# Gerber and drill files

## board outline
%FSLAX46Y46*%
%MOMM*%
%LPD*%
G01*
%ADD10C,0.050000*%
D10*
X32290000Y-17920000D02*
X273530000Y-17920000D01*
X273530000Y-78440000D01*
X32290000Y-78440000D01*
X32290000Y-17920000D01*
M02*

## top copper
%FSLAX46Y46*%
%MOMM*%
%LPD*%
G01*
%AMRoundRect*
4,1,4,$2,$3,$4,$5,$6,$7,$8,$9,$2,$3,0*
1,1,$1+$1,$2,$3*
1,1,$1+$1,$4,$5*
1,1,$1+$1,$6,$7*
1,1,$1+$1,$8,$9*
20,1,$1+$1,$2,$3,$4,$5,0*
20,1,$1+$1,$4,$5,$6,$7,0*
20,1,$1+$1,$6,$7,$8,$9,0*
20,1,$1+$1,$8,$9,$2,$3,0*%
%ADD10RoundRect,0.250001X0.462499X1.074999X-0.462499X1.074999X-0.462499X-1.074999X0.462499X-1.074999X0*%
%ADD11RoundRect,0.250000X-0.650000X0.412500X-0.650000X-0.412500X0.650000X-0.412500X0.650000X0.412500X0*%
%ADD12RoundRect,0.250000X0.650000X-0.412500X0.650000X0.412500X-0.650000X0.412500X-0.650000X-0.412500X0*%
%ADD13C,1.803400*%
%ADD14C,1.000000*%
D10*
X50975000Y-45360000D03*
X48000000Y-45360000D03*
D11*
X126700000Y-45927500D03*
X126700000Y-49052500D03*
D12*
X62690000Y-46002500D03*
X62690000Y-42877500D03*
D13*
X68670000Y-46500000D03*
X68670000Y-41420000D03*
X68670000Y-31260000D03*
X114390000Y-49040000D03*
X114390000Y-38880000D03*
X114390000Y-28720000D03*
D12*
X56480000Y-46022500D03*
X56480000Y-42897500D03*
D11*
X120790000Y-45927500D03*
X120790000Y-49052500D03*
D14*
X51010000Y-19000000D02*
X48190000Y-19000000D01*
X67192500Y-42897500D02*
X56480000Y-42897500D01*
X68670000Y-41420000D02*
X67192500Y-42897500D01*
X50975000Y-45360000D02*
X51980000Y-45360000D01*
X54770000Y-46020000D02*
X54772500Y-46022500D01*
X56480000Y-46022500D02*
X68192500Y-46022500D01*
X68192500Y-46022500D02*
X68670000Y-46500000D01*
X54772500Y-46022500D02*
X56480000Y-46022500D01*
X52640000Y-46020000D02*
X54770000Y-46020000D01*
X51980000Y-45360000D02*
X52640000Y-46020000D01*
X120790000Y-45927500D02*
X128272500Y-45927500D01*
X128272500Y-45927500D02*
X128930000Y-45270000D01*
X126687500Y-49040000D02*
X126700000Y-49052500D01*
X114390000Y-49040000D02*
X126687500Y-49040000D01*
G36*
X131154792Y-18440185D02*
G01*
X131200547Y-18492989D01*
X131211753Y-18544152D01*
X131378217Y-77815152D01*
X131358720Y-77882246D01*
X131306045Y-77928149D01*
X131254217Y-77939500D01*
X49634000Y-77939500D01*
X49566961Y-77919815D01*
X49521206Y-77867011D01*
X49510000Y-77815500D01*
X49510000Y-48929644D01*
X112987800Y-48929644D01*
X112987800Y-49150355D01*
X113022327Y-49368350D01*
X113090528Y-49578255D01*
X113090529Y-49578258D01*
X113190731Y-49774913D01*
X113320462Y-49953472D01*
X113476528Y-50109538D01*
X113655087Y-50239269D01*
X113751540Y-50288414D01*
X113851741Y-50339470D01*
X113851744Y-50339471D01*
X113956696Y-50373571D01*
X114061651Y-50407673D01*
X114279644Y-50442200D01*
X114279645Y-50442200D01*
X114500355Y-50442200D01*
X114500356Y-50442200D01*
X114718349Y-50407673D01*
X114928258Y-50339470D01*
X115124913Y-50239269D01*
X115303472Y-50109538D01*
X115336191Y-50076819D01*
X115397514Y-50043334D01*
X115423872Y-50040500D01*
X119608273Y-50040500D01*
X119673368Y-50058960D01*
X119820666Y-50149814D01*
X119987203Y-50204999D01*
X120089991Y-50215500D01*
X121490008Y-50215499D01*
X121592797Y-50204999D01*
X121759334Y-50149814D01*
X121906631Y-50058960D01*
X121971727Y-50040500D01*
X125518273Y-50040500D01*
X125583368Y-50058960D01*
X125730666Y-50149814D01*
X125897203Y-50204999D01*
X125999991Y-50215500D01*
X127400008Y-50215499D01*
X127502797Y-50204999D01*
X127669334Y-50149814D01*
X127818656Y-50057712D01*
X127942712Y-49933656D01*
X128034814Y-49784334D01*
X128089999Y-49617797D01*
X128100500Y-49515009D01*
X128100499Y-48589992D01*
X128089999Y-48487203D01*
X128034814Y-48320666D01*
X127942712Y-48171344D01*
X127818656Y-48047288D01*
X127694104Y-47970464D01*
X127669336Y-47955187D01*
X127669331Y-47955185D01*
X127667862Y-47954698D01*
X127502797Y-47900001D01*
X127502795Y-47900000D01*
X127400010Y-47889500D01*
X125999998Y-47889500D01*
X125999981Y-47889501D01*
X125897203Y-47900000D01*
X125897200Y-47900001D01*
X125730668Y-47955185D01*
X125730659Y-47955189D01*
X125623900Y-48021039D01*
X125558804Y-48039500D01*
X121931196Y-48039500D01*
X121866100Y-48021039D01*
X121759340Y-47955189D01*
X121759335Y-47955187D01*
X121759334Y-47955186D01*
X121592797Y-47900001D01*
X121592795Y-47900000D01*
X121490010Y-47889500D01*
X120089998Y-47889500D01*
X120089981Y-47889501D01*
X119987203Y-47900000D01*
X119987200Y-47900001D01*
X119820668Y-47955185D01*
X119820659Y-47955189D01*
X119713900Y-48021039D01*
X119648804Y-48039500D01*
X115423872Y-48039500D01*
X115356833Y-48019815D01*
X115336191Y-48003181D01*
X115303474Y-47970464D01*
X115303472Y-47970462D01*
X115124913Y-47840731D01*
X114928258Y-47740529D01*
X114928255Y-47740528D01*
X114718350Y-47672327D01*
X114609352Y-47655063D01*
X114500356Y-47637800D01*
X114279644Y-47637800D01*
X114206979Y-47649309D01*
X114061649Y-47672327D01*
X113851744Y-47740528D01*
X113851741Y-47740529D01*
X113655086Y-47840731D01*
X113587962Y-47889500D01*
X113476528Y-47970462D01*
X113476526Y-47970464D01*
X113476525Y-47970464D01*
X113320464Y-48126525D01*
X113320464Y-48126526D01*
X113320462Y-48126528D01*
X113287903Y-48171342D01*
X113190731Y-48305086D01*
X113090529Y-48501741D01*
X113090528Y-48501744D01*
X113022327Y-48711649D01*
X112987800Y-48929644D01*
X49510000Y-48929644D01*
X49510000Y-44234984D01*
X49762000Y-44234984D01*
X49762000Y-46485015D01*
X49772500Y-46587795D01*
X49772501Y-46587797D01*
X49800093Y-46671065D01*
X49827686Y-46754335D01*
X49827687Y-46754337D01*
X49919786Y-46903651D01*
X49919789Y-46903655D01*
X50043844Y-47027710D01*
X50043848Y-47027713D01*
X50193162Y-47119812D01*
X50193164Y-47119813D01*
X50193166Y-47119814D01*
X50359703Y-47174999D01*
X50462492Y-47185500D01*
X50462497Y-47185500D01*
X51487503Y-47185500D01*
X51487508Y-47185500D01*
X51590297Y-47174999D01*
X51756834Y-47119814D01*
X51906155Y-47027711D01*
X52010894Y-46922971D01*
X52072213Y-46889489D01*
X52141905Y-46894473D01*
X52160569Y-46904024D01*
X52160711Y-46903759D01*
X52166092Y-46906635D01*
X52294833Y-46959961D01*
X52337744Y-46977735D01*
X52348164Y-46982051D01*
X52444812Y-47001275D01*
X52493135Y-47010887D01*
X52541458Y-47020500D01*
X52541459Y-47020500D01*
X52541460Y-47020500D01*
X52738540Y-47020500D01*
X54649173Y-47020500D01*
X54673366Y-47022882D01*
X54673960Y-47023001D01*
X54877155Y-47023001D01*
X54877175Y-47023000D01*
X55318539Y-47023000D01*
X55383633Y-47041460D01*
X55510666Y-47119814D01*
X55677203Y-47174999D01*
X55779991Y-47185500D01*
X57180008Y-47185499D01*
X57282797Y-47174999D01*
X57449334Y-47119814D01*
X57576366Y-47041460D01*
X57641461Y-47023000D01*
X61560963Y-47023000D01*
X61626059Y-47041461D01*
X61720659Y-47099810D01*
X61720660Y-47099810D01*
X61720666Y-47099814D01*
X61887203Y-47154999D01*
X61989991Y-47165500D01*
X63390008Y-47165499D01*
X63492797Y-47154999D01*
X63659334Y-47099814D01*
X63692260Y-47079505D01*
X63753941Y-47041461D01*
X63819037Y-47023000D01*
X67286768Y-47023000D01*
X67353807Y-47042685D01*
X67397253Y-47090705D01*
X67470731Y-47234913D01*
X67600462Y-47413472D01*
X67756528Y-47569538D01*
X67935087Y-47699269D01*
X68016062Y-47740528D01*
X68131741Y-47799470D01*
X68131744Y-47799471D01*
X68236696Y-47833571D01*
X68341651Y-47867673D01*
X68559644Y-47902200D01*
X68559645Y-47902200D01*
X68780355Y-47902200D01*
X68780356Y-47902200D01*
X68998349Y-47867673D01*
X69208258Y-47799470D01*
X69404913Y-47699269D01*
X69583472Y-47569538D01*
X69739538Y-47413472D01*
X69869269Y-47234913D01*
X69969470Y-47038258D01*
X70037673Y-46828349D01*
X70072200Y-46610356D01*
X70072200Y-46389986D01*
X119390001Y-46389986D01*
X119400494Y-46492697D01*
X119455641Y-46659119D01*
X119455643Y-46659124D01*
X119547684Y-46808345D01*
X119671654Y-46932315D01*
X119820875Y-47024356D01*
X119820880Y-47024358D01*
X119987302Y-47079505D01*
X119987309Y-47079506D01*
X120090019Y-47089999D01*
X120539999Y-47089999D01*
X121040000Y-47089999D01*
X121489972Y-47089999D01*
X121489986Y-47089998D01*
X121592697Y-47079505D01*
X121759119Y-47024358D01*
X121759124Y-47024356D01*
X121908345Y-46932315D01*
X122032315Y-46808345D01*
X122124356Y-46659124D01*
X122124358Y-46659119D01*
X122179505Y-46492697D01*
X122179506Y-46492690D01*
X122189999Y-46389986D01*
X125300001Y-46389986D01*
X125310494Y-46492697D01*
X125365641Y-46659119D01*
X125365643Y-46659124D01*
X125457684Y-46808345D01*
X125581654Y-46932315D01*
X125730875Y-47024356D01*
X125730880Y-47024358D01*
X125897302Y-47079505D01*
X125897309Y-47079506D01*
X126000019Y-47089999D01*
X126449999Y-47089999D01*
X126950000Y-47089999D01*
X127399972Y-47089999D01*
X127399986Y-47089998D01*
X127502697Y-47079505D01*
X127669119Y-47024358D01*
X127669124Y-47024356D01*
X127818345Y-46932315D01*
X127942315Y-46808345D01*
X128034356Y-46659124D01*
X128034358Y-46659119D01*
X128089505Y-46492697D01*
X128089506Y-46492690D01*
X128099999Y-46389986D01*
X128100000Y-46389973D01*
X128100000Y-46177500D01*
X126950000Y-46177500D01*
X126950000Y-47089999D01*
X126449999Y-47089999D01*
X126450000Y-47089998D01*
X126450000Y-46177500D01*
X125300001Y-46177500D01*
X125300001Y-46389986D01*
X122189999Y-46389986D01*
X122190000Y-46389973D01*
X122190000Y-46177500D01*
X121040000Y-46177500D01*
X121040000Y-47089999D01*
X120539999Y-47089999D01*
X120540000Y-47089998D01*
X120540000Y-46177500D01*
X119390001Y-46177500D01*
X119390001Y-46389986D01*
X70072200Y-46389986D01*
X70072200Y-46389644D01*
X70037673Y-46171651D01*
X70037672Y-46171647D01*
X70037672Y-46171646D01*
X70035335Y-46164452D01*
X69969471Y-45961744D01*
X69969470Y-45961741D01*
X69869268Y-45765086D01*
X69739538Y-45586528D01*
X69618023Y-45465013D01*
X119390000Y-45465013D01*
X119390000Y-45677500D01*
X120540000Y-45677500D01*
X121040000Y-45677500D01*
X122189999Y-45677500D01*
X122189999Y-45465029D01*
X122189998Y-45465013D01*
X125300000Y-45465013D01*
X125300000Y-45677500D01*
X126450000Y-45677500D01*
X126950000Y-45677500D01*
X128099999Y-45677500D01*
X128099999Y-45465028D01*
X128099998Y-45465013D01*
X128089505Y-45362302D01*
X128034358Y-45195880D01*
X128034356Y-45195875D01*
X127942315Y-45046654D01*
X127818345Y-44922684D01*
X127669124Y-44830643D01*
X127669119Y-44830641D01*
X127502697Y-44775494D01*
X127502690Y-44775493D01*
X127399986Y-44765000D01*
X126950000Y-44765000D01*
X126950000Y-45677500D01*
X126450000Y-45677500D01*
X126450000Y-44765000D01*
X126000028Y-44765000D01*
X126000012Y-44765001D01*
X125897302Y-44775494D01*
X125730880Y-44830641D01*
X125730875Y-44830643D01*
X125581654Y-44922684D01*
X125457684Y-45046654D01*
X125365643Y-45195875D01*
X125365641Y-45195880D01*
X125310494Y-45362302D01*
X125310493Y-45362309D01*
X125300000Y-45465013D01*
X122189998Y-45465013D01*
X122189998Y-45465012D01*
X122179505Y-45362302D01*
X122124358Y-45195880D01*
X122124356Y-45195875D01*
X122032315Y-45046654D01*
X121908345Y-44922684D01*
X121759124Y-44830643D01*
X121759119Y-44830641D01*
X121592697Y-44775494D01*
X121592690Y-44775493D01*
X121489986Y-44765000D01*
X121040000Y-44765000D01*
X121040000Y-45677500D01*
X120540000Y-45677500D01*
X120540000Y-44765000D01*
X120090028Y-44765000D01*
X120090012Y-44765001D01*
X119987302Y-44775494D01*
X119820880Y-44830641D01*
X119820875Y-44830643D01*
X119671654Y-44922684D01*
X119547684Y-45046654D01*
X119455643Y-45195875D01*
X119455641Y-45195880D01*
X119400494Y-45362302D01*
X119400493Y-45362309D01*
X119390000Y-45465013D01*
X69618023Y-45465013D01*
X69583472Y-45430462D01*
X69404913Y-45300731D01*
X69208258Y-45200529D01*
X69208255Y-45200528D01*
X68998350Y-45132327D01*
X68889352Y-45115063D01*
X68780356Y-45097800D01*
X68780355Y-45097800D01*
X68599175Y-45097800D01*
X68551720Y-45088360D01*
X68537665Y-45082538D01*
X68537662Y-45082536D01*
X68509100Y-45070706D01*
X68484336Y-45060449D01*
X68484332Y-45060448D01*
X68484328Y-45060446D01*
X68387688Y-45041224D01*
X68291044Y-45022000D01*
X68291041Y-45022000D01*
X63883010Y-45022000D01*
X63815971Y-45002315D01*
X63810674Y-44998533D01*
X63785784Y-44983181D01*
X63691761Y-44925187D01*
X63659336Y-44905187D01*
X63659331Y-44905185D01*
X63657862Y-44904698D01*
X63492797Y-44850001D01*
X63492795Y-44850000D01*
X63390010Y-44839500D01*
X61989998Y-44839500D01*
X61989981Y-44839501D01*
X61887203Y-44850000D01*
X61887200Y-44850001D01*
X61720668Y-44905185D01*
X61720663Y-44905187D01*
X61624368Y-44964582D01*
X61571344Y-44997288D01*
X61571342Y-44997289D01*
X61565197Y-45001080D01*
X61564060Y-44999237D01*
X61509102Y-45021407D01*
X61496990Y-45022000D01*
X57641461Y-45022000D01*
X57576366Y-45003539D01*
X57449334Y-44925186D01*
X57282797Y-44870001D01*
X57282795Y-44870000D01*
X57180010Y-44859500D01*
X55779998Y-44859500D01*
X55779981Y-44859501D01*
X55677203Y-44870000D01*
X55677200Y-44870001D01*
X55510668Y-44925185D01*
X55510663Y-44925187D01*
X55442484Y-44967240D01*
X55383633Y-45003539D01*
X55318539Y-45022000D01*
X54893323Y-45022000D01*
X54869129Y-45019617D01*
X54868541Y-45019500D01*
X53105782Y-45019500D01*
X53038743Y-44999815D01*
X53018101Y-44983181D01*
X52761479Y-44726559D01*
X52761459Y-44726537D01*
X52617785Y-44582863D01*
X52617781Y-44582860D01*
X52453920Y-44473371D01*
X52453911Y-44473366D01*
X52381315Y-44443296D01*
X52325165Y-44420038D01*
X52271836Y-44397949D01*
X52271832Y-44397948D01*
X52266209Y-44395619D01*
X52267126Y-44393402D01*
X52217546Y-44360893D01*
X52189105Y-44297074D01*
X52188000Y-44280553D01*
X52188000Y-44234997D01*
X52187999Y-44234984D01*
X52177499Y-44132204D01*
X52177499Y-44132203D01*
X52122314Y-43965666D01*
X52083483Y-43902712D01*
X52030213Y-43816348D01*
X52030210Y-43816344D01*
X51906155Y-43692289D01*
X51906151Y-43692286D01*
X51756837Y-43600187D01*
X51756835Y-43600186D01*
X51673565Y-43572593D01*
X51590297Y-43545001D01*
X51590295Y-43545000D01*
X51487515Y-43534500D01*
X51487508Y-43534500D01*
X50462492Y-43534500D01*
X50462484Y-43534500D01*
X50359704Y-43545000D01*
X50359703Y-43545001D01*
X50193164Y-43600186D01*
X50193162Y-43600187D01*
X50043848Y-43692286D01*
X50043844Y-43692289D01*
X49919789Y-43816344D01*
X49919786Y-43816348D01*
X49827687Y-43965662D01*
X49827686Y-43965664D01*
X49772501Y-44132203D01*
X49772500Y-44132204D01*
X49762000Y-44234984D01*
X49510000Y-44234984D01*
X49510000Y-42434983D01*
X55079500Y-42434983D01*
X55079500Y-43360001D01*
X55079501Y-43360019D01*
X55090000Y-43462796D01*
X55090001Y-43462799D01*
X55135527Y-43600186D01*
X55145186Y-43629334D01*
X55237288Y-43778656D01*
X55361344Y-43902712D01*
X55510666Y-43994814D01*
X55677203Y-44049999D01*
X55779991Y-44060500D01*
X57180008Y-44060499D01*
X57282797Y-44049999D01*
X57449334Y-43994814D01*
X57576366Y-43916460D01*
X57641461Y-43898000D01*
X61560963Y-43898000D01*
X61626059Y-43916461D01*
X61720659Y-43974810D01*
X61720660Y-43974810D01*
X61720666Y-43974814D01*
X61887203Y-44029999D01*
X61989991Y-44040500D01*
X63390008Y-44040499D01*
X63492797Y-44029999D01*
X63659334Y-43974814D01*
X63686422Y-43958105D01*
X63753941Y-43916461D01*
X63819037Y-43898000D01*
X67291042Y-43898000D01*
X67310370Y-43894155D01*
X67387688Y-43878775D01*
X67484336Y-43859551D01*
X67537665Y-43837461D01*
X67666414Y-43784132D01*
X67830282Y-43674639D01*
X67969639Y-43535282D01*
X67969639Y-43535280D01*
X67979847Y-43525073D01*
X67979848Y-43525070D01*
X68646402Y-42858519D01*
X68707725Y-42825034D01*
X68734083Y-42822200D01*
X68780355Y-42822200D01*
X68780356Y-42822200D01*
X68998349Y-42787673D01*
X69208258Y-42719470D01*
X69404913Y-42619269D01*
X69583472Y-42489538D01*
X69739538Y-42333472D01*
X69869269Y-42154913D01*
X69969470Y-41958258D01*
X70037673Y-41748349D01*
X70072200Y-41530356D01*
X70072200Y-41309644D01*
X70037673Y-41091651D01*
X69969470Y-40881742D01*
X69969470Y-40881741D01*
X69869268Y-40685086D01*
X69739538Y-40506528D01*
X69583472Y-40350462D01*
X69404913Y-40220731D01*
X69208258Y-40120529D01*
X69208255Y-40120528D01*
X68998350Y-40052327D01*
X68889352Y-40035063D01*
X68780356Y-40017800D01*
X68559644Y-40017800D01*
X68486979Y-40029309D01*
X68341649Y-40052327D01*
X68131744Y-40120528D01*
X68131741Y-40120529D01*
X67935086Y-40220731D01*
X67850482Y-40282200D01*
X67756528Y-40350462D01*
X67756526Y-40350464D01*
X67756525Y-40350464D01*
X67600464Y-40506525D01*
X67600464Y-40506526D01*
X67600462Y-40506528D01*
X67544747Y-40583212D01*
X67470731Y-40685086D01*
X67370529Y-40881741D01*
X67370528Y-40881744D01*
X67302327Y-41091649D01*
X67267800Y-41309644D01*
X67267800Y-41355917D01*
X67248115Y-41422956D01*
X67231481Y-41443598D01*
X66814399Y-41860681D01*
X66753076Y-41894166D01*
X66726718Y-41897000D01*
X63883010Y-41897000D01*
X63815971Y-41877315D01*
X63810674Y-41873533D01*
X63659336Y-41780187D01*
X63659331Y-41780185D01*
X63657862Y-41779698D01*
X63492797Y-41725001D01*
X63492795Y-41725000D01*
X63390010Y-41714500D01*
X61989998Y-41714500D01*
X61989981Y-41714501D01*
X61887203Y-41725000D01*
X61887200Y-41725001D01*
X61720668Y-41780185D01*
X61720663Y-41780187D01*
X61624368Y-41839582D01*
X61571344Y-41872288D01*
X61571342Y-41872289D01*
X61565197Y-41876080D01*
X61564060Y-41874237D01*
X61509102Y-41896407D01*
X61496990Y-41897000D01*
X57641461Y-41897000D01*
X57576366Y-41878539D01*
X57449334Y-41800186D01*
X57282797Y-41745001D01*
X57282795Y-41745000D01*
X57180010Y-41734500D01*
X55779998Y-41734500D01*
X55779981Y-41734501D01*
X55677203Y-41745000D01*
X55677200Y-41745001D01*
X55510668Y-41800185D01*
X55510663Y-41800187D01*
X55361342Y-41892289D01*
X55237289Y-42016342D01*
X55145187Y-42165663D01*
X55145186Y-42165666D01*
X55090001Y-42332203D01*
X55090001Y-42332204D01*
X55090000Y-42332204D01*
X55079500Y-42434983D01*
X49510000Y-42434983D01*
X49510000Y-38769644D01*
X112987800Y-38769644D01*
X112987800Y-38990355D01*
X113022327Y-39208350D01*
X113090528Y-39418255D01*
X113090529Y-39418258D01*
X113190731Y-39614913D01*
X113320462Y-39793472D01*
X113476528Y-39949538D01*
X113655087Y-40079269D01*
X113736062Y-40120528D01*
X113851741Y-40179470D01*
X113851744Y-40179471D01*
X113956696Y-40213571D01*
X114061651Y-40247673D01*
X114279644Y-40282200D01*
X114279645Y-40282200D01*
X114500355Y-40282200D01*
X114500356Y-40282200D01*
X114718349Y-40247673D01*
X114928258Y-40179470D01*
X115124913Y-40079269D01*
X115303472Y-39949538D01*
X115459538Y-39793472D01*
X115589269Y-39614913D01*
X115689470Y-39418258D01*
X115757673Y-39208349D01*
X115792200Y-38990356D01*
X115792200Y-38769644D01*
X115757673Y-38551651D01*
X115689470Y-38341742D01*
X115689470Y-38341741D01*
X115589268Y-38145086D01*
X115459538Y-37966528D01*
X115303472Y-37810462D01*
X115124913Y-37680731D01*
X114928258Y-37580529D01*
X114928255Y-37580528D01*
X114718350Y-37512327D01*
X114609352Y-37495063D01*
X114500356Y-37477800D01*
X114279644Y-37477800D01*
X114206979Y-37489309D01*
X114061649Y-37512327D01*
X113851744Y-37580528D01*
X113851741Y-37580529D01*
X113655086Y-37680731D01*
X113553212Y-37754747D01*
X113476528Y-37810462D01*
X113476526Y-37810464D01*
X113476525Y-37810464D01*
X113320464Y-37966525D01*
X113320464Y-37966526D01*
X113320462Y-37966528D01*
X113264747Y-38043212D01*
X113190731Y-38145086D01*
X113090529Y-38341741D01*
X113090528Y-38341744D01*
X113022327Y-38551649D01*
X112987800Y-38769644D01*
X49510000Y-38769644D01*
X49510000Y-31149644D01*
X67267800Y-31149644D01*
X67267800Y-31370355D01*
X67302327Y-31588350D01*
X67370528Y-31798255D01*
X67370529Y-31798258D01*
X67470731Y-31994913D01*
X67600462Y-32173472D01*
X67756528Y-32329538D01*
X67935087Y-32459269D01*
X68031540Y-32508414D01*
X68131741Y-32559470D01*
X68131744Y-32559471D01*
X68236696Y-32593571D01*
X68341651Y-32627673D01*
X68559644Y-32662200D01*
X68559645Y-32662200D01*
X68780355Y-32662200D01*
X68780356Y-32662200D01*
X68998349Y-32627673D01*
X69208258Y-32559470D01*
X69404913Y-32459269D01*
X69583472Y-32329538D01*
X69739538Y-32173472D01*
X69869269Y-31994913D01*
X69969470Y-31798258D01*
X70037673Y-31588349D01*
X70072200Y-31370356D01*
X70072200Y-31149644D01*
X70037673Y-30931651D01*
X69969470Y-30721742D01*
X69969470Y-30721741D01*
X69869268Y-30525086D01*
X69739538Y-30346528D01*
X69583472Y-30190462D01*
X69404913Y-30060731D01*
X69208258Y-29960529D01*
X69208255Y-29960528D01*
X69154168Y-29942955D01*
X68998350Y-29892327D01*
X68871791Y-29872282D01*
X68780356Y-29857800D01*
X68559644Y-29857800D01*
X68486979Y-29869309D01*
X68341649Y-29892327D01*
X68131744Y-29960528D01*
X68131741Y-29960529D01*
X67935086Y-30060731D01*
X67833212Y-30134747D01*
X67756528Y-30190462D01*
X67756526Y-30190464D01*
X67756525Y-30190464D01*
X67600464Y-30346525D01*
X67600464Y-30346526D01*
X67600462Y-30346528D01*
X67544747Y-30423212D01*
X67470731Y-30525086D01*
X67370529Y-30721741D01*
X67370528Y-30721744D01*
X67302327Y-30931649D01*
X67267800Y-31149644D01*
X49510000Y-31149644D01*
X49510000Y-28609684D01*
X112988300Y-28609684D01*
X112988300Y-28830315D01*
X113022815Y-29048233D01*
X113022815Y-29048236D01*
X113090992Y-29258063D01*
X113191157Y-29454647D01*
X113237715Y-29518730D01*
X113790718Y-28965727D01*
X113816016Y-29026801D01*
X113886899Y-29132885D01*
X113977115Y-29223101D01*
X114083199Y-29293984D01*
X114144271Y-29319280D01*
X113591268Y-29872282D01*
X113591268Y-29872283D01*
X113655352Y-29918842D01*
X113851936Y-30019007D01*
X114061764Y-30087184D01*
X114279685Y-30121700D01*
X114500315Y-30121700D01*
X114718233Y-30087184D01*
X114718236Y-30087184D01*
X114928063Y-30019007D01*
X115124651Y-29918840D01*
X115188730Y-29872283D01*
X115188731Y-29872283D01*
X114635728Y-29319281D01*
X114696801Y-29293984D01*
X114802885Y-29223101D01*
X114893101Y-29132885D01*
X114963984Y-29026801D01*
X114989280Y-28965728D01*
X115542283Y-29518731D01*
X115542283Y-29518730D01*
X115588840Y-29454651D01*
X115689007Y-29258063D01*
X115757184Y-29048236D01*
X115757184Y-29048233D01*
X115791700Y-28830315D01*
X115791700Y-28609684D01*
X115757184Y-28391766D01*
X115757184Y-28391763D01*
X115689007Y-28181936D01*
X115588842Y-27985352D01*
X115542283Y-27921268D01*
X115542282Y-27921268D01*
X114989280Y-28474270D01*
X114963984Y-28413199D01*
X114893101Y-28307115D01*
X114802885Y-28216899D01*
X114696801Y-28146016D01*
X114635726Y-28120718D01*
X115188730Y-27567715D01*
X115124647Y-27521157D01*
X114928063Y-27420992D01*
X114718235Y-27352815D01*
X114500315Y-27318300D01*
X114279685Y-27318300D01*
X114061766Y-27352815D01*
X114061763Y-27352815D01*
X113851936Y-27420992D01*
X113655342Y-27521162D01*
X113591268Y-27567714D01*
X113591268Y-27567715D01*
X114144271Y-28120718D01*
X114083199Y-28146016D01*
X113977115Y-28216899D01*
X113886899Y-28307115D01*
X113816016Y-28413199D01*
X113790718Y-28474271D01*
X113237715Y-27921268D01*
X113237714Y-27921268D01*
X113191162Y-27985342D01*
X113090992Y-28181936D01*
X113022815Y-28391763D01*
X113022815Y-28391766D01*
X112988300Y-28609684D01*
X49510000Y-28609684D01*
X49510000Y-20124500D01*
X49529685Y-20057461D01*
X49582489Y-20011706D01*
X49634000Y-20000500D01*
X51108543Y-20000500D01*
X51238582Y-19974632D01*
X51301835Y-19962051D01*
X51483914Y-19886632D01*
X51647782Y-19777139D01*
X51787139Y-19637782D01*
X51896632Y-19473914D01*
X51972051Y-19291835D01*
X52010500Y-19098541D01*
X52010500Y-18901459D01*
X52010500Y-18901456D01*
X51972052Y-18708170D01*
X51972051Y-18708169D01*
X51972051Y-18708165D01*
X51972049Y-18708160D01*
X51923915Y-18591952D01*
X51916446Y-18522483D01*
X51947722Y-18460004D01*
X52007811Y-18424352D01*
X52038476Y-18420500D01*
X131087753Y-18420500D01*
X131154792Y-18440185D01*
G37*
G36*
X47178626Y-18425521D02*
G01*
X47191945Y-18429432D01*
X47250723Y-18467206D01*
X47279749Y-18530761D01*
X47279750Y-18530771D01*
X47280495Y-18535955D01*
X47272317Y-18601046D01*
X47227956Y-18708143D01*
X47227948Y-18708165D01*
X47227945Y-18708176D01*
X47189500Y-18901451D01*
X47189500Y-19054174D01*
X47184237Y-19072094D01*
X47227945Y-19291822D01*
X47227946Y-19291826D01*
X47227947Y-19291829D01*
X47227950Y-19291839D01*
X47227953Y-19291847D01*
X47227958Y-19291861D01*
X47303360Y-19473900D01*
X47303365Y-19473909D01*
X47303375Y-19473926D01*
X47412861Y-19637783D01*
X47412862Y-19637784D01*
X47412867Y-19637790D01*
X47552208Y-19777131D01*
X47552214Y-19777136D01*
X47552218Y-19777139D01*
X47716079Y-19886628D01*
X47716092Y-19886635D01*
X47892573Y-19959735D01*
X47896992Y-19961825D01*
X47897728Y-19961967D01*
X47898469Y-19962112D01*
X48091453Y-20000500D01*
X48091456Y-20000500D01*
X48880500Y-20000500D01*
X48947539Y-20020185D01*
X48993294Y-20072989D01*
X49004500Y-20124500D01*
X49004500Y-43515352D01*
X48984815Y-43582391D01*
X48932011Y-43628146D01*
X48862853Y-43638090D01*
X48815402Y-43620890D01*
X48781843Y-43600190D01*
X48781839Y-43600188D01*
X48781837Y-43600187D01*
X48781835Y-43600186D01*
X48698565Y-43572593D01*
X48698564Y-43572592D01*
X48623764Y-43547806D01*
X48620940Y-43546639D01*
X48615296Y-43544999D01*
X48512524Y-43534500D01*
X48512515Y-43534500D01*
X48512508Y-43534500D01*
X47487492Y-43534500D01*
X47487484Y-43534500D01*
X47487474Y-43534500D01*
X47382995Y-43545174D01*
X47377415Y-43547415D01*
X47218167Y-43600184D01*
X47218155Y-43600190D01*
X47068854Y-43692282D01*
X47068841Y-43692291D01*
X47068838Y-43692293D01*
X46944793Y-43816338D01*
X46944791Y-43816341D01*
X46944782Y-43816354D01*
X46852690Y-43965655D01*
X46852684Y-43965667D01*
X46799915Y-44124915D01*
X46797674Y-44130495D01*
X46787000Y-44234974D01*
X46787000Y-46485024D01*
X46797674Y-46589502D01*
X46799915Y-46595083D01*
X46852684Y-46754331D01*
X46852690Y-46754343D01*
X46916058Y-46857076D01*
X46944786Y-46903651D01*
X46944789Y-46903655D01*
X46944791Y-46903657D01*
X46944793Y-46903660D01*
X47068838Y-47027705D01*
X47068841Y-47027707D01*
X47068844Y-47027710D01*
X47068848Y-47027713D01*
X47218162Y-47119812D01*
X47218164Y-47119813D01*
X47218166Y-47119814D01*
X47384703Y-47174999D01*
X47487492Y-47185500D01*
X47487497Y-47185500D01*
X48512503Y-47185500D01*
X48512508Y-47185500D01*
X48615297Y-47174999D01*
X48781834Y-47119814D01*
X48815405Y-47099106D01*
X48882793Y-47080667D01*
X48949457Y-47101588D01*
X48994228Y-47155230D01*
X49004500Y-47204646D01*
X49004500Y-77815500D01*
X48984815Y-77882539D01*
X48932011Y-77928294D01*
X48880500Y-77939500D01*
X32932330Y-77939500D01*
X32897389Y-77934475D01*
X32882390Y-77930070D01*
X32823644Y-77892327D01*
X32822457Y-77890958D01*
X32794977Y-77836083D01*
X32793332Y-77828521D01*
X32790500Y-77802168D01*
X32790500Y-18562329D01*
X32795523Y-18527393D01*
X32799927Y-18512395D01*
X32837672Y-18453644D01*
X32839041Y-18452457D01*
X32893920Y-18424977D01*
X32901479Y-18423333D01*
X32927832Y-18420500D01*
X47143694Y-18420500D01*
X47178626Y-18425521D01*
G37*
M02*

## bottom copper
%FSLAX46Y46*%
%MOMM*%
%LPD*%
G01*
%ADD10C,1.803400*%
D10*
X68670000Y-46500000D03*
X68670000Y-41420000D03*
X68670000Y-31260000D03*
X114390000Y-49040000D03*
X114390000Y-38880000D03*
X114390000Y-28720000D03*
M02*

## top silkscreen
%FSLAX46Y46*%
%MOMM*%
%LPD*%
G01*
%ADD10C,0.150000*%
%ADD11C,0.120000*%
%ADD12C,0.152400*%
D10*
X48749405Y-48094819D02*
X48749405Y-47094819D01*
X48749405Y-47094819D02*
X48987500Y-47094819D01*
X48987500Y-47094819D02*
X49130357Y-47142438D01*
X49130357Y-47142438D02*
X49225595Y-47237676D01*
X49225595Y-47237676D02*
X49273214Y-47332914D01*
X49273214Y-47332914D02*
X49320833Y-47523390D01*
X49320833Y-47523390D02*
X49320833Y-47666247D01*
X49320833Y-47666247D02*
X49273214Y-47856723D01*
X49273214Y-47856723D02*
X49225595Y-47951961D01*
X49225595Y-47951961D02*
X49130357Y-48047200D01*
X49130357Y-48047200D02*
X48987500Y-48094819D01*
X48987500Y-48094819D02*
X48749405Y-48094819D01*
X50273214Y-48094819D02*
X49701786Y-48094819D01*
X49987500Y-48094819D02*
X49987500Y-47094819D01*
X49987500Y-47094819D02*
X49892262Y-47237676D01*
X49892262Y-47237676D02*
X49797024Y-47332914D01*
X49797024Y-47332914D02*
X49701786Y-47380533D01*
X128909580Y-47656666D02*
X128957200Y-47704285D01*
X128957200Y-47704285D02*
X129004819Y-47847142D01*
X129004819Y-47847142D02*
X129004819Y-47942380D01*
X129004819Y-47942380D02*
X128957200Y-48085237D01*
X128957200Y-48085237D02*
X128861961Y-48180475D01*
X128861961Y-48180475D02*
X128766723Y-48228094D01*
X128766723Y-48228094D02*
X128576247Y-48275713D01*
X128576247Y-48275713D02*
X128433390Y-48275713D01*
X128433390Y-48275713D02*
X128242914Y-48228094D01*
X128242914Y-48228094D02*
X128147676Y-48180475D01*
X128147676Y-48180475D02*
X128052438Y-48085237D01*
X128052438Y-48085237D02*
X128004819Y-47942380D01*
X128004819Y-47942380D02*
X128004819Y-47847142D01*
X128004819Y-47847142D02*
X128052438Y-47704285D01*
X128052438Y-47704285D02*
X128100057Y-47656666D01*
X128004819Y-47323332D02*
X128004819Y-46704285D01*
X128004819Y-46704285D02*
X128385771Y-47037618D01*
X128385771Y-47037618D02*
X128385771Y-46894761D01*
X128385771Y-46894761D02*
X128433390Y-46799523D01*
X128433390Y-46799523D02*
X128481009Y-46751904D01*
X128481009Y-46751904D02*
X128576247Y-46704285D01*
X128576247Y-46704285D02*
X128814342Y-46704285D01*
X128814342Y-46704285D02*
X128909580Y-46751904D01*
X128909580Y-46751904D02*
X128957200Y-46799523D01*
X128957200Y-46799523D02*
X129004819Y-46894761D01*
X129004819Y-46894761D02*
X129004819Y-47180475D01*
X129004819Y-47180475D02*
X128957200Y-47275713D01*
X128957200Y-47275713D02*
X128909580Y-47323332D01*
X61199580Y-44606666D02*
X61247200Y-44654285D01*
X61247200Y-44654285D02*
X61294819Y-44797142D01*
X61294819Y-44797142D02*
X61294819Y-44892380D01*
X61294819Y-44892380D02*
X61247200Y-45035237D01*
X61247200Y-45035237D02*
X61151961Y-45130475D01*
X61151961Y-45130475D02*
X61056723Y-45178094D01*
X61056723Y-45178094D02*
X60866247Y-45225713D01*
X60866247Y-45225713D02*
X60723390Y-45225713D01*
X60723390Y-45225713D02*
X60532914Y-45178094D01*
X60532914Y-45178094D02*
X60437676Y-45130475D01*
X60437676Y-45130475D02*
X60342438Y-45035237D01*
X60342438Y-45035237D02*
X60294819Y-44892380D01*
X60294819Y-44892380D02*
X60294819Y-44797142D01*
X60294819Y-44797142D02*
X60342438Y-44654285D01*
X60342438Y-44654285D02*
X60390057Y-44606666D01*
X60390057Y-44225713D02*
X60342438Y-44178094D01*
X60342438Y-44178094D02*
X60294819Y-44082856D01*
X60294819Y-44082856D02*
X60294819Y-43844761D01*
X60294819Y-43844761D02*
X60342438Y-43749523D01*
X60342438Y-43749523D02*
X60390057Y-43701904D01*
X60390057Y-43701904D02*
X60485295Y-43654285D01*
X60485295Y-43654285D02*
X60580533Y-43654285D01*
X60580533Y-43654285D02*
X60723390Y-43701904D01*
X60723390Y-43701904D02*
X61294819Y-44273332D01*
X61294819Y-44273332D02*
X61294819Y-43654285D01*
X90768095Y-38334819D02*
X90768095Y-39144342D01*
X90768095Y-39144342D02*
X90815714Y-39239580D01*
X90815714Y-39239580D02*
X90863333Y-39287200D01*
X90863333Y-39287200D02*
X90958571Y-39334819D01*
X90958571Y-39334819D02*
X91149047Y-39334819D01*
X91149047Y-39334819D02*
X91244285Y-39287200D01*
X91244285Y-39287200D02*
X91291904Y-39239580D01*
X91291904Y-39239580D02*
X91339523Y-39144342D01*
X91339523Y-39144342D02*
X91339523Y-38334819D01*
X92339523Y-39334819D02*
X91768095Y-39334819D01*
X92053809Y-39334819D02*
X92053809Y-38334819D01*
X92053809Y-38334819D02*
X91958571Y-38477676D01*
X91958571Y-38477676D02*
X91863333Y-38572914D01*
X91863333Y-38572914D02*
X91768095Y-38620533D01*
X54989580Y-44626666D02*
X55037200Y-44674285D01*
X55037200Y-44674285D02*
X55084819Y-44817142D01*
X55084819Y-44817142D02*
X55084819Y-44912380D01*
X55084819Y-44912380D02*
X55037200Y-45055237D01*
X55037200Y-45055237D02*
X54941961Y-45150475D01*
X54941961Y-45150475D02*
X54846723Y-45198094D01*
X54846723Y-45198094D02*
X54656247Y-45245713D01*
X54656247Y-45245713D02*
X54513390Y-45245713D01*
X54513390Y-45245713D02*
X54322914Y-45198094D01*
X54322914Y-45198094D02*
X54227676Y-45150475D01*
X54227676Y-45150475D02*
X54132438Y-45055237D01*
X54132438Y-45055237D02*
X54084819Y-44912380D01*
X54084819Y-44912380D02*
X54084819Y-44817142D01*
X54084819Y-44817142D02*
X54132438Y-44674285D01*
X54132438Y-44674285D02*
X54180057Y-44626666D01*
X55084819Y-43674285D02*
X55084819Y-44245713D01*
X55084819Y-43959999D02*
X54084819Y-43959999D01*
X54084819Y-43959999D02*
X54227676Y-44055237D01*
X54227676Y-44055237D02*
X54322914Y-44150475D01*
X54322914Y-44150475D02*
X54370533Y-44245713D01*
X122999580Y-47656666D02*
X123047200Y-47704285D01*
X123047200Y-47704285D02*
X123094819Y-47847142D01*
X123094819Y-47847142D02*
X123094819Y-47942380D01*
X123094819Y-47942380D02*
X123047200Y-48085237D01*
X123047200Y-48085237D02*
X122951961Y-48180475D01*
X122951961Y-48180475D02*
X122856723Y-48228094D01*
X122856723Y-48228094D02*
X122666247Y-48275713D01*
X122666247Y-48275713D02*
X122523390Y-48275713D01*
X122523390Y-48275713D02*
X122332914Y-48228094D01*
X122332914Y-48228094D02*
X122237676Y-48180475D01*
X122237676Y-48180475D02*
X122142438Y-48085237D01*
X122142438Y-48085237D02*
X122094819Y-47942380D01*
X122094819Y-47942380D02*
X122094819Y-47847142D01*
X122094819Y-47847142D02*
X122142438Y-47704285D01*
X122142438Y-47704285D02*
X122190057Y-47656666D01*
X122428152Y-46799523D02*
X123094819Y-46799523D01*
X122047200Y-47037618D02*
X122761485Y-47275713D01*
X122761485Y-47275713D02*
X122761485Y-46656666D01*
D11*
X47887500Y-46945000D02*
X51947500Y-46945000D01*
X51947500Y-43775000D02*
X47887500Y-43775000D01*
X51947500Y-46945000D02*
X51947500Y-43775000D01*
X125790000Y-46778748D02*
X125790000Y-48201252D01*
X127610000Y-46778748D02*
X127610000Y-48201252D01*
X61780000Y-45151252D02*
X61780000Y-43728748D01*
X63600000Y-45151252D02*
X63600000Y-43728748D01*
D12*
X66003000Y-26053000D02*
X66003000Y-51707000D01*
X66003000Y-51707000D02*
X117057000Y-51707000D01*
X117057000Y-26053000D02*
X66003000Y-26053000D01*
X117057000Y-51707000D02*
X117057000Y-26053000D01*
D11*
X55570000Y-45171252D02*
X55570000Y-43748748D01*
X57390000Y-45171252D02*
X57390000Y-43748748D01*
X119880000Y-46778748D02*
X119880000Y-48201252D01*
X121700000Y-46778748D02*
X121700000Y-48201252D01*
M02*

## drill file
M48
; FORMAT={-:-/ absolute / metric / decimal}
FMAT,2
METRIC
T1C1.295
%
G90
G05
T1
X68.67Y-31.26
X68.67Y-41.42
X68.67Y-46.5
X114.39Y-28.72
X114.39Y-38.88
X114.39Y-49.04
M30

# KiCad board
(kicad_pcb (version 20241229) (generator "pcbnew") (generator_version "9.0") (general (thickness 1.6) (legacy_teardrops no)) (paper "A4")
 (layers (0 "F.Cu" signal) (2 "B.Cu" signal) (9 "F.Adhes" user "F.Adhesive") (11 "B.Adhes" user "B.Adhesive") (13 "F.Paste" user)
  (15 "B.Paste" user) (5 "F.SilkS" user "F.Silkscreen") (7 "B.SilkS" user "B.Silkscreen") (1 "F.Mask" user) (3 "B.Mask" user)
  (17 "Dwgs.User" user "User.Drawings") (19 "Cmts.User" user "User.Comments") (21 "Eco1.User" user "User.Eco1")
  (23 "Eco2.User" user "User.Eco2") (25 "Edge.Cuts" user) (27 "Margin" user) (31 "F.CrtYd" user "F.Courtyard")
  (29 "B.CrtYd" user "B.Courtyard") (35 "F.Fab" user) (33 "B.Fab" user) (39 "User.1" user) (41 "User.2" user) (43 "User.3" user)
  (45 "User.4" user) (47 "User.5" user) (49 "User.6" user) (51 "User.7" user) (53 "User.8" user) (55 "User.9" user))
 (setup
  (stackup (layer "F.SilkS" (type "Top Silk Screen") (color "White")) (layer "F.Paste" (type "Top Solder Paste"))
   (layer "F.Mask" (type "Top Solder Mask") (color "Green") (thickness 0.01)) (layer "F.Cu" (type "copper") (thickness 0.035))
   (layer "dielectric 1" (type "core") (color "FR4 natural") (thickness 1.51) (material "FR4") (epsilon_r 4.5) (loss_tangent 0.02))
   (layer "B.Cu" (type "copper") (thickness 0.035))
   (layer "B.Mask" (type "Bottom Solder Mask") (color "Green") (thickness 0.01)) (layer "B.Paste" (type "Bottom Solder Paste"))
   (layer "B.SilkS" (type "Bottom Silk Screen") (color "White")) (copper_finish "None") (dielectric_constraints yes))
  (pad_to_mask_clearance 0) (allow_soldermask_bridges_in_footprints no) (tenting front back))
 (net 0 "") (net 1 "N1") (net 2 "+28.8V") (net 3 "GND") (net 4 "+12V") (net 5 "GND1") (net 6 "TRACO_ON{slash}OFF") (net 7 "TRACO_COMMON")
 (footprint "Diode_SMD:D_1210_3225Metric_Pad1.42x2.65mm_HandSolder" (layer "F.Cu") (at 49.4875 45.36 180)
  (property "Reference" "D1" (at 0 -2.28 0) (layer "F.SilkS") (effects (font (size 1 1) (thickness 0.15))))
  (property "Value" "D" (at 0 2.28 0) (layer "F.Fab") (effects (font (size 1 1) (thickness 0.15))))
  (fp_line (start 1.6 -1.585) (end -2.46 -1.585) (stroke (width 0.12) (type solid)) (layer "F.SilkS"))
  (fp_line (start -2.46 1.585) (end 1.6 1.585) (stroke (width 0.12) (type solid)) (layer "F.SilkS"))
  (fp_line (start -2.46 -1.585) (end -2.46 1.585) (stroke (width 0.12) (type solid)) (layer "F.SilkS"))
  (pad "1" smd roundrect (at -1.4875 0 180) (size 1.425 2.65) (layers "F.Cu" "F.Mask" "F.Paste") (roundrect_rratio 0.175439) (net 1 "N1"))
  (pad "2" smd roundrect (at 1.4875 0 180) (size 1.425 2.65) (layers "F.Cu" "F.Mask" "F.Paste") (roundrect_rratio 0.175439) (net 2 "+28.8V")))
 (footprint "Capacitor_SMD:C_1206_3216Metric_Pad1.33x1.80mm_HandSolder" (layer "F.Cu") (at 126.7 47.49 -90)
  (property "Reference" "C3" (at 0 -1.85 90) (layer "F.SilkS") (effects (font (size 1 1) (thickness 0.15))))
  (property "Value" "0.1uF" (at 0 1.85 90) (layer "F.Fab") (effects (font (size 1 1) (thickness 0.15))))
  (fp_line (start -0.711252 0.91) (end 0.711252 0.91) (stroke (width 0.12) (type solid)) (layer "F.SilkS"))
  (fp_line (start -0.711252 -0.91) (end 0.711252 -0.91) (stroke (width 0.12) (type solid)) (layer "F.SilkS"))
  (pad "1" smd roundrect (at -1.5625 0 270) (size 1.325 1.8) (layers "F.Cu" "F.Mask" "F.Paste") (roundrect_rratio 0.188679) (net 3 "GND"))
  (pad "2" smd roundrect (at 1.5625 0 270) (size 1.325 1.8) (layers "F.Cu" "F.Mask" "F.Paste") (roundrect_rratio 0.188679) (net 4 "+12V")))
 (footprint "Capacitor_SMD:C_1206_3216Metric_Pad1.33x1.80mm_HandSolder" (layer "F.Cu") (at 62.69 44.44 90)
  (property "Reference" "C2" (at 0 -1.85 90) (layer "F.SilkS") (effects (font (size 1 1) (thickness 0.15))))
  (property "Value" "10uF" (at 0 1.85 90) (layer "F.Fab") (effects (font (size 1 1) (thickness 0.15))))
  (fp_line (start -0.711252 -0.91) (end 0.711252 -0.91) (stroke (width 0.12) (type solid)) (layer "F.SilkS"))
  (fp_line (start -0.711252 0.91) (end 0.711252 0.91) (stroke (width 0.12) (type solid)) (layer "F.SilkS"))
  (pad "1" smd roundrect (at -1.5625 0 90) (size 1.325 1.8) (layers "F.Cu" "F.Mask" "F.Paste") (roundrect_rratio 0.188679) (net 1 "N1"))
  (pad "2" smd roundrect (at 1.5625 0 90) (size 1.325 1.8) (layers "F.Cu" "F.Mask" "F.Paste") (roundrect_rratio 0.188679) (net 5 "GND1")))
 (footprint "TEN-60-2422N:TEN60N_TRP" (layer "F.Cu") (at 68.67 46.5)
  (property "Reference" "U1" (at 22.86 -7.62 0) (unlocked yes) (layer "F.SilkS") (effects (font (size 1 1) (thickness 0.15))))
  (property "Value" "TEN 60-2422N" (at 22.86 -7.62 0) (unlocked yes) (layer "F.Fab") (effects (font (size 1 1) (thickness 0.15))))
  (fp_line (start -2.667 -20.447) (end -2.667 5.207) (stroke (width 0.1524) (type solid)) (layer "F.SilkS"))
  (fp_line (start -2.667 5.207) (end 48.387 5.207) (stroke (width 0.1524) (type solid)) (layer "F.SilkS"))
  (fp_line (start 48.387 -20.447) (end -2.667 -20.447) (stroke (width 0.1524) (type solid)) (layer "F.SilkS"))
  (fp_line (start 48.387 5.207) (end 48.387 -20.447) (stroke (width 0.1524) (type solid)) (layer "F.SilkS"))
  (pad "1" thru_hole circle (at 0 0) (size 1.8034 1.8034) (drill 1.2954) (layers "*.Cu" "*.Mask") (remove_unused_layers no) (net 1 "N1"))
  (pad "2" thru_hole circle (at 0 -5.08) (size 1.8034 1.8034) (drill 1.2954) (layers "*.Cu" "*.Mask") (remove_unused_layers no)
   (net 5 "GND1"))
  (pad "3" thru_hole circle (at 0 -15.24) (size 1.8034 1.8034) (drill 1.2954) (layers "*.Cu" "*.Mask") (remove_unused_layers no)
   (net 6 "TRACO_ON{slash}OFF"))
  (pad "4" thru_hole circle (at 45.72 2.54) (size 1.8034 1.8034) (drill 1.2954) (layers "*.Cu" "*.Mask") (remove_unused_layers no)
   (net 4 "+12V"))
  (pad "5" thru_hole circle (at 45.72 -7.62) (size 1.8034 1.8034) (drill 1.2954) (layers "*.Cu" "*.Mask") (remove_unused_layers no)
   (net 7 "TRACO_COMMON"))
  (pad "6" thru_hole circle (at 45.72 -17.78) (size 1.8034 1.8034) (drill 1.2954) (layers "*.Cu" "*.Mask") (remove_unused_layers no)
   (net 3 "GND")))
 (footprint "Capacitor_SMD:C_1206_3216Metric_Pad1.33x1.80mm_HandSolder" (layer "F.Cu") (at 56.48 44.46 90)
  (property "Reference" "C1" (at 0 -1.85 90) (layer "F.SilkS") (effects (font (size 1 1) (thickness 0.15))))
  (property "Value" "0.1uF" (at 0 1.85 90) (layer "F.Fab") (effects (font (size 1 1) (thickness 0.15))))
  (fp_line (start -0.711252 -0.91) (end 0.711252 -0.91) (stroke (width 0.12) (type solid)) (layer "F.SilkS"))
  (fp_line (start -0.711252 0.91) (end 0.711252 0.91) (stroke (width 0.12) (type solid)) (layer "F.SilkS"))
  (pad "1" smd roundrect (at -1.5625 0 90) (size 1.325 1.8) (layers "F.Cu" "F.Mask" "F.Paste") (roundrect_rratio 0.188679) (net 1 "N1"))
  (pad "2" smd roundrect (at 1.5625 0 90) (size 1.325 1.8) (layers "F.Cu" "F.Mask" "F.Paste") (roundrect_rratio 0.188679) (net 5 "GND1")))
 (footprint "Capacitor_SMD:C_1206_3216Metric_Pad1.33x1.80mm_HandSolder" (layer "F.Cu") (at 120.79 47.49 -90)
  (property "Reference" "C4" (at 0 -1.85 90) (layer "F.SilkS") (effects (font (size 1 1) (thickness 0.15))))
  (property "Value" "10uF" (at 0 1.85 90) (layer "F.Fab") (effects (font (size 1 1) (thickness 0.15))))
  (fp_line (start -0.711252 0.91) (end 0.711252 0.91) (stroke (width 0.12) (type solid)) (layer "F.SilkS"))
  (fp_line (start -0.711252 -0.91) (end 0.711252 -0.91) (stroke (width 0.12) (type solid)) (layer "F.SilkS"))
  (pad "1" smd roundrect (at -1.5625 0 270) (size 1.325 1.8) (layers "F.Cu" "F.Mask" "F.Paste") (roundrect_rratio 0.188679) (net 3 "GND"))
  (pad "2" smd roundrect (at 1.5625 0 270) (size 1.325 1.8) (layers "F.Cu" "F.Mask" "F.Paste") (roundrect_rratio 0.188679) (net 4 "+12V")))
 (gr_rect (start 32.29 17.92) (end 273.53 78.44) (stroke (width 0.05) (type default)) (fill no) (layer "Edge.Cuts"))
 (segment (start 51.01 19) (end 48.19 19) (width 1) (layer "F.Cu") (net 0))
 (segment (start 67.1925 42.8975) (end 56.48 42.8975) (width 1) (layer "F.Cu") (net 5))
 (segment (start 68.67 41.42) (end 67.1925 42.8975) (width 1) (layer "F.Cu") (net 5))
 (segment (start 50.975 45.36) (end 51.98 45.36) (width 1) (layer "F.Cu") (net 1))
 (segment (start 54.77 46.02) (end 54.7725 46.0225) (width 1) (layer "F.Cu") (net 1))
 (segment (start 56.48 46.0225) (end 68.1925 46.0225) (width 1) (layer "F.Cu") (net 1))
 (segment (start 68.1925 46.0225) (end 68.67 46.5) (width 1) (layer "F.Cu") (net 1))
 (segment (start 54.7725 46.0225) (end 56.48 46.0225) (width 1) (layer "F.Cu") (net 1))
 (segment (start 52.64 46.02) (end 54.77 46.02) (width 1) (layer "F.Cu") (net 1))
 (segment (start 51.98 45.36) (end 52.64 46.02) (width 1) (layer "F.Cu") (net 1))
 (segment (start 120.79 45.9275) (end 128.2725 45.9275) (width 1) (layer "F.Cu") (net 3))
 (segment (start 128.2725 45.9275) (end 128.93 45.27) (width 1) (layer "F.Cu") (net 3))
 (segment (start 126.6875 49.04) (end 126.7 49.0525) (width 1) (layer "F.Cu") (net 4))
 (segment (start 114.39 49.04) (end 126.6875 49.04) (width 1) (layer "F.Cu") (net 4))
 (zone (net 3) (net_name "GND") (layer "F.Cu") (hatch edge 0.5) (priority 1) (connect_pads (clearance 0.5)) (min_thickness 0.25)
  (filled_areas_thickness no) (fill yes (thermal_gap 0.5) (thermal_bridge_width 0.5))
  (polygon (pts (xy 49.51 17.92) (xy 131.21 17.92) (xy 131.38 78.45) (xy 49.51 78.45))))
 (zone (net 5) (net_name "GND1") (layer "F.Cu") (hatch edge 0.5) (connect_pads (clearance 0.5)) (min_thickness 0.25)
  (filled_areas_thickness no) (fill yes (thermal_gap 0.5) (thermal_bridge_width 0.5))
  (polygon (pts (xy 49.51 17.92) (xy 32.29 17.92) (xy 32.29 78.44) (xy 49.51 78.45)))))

